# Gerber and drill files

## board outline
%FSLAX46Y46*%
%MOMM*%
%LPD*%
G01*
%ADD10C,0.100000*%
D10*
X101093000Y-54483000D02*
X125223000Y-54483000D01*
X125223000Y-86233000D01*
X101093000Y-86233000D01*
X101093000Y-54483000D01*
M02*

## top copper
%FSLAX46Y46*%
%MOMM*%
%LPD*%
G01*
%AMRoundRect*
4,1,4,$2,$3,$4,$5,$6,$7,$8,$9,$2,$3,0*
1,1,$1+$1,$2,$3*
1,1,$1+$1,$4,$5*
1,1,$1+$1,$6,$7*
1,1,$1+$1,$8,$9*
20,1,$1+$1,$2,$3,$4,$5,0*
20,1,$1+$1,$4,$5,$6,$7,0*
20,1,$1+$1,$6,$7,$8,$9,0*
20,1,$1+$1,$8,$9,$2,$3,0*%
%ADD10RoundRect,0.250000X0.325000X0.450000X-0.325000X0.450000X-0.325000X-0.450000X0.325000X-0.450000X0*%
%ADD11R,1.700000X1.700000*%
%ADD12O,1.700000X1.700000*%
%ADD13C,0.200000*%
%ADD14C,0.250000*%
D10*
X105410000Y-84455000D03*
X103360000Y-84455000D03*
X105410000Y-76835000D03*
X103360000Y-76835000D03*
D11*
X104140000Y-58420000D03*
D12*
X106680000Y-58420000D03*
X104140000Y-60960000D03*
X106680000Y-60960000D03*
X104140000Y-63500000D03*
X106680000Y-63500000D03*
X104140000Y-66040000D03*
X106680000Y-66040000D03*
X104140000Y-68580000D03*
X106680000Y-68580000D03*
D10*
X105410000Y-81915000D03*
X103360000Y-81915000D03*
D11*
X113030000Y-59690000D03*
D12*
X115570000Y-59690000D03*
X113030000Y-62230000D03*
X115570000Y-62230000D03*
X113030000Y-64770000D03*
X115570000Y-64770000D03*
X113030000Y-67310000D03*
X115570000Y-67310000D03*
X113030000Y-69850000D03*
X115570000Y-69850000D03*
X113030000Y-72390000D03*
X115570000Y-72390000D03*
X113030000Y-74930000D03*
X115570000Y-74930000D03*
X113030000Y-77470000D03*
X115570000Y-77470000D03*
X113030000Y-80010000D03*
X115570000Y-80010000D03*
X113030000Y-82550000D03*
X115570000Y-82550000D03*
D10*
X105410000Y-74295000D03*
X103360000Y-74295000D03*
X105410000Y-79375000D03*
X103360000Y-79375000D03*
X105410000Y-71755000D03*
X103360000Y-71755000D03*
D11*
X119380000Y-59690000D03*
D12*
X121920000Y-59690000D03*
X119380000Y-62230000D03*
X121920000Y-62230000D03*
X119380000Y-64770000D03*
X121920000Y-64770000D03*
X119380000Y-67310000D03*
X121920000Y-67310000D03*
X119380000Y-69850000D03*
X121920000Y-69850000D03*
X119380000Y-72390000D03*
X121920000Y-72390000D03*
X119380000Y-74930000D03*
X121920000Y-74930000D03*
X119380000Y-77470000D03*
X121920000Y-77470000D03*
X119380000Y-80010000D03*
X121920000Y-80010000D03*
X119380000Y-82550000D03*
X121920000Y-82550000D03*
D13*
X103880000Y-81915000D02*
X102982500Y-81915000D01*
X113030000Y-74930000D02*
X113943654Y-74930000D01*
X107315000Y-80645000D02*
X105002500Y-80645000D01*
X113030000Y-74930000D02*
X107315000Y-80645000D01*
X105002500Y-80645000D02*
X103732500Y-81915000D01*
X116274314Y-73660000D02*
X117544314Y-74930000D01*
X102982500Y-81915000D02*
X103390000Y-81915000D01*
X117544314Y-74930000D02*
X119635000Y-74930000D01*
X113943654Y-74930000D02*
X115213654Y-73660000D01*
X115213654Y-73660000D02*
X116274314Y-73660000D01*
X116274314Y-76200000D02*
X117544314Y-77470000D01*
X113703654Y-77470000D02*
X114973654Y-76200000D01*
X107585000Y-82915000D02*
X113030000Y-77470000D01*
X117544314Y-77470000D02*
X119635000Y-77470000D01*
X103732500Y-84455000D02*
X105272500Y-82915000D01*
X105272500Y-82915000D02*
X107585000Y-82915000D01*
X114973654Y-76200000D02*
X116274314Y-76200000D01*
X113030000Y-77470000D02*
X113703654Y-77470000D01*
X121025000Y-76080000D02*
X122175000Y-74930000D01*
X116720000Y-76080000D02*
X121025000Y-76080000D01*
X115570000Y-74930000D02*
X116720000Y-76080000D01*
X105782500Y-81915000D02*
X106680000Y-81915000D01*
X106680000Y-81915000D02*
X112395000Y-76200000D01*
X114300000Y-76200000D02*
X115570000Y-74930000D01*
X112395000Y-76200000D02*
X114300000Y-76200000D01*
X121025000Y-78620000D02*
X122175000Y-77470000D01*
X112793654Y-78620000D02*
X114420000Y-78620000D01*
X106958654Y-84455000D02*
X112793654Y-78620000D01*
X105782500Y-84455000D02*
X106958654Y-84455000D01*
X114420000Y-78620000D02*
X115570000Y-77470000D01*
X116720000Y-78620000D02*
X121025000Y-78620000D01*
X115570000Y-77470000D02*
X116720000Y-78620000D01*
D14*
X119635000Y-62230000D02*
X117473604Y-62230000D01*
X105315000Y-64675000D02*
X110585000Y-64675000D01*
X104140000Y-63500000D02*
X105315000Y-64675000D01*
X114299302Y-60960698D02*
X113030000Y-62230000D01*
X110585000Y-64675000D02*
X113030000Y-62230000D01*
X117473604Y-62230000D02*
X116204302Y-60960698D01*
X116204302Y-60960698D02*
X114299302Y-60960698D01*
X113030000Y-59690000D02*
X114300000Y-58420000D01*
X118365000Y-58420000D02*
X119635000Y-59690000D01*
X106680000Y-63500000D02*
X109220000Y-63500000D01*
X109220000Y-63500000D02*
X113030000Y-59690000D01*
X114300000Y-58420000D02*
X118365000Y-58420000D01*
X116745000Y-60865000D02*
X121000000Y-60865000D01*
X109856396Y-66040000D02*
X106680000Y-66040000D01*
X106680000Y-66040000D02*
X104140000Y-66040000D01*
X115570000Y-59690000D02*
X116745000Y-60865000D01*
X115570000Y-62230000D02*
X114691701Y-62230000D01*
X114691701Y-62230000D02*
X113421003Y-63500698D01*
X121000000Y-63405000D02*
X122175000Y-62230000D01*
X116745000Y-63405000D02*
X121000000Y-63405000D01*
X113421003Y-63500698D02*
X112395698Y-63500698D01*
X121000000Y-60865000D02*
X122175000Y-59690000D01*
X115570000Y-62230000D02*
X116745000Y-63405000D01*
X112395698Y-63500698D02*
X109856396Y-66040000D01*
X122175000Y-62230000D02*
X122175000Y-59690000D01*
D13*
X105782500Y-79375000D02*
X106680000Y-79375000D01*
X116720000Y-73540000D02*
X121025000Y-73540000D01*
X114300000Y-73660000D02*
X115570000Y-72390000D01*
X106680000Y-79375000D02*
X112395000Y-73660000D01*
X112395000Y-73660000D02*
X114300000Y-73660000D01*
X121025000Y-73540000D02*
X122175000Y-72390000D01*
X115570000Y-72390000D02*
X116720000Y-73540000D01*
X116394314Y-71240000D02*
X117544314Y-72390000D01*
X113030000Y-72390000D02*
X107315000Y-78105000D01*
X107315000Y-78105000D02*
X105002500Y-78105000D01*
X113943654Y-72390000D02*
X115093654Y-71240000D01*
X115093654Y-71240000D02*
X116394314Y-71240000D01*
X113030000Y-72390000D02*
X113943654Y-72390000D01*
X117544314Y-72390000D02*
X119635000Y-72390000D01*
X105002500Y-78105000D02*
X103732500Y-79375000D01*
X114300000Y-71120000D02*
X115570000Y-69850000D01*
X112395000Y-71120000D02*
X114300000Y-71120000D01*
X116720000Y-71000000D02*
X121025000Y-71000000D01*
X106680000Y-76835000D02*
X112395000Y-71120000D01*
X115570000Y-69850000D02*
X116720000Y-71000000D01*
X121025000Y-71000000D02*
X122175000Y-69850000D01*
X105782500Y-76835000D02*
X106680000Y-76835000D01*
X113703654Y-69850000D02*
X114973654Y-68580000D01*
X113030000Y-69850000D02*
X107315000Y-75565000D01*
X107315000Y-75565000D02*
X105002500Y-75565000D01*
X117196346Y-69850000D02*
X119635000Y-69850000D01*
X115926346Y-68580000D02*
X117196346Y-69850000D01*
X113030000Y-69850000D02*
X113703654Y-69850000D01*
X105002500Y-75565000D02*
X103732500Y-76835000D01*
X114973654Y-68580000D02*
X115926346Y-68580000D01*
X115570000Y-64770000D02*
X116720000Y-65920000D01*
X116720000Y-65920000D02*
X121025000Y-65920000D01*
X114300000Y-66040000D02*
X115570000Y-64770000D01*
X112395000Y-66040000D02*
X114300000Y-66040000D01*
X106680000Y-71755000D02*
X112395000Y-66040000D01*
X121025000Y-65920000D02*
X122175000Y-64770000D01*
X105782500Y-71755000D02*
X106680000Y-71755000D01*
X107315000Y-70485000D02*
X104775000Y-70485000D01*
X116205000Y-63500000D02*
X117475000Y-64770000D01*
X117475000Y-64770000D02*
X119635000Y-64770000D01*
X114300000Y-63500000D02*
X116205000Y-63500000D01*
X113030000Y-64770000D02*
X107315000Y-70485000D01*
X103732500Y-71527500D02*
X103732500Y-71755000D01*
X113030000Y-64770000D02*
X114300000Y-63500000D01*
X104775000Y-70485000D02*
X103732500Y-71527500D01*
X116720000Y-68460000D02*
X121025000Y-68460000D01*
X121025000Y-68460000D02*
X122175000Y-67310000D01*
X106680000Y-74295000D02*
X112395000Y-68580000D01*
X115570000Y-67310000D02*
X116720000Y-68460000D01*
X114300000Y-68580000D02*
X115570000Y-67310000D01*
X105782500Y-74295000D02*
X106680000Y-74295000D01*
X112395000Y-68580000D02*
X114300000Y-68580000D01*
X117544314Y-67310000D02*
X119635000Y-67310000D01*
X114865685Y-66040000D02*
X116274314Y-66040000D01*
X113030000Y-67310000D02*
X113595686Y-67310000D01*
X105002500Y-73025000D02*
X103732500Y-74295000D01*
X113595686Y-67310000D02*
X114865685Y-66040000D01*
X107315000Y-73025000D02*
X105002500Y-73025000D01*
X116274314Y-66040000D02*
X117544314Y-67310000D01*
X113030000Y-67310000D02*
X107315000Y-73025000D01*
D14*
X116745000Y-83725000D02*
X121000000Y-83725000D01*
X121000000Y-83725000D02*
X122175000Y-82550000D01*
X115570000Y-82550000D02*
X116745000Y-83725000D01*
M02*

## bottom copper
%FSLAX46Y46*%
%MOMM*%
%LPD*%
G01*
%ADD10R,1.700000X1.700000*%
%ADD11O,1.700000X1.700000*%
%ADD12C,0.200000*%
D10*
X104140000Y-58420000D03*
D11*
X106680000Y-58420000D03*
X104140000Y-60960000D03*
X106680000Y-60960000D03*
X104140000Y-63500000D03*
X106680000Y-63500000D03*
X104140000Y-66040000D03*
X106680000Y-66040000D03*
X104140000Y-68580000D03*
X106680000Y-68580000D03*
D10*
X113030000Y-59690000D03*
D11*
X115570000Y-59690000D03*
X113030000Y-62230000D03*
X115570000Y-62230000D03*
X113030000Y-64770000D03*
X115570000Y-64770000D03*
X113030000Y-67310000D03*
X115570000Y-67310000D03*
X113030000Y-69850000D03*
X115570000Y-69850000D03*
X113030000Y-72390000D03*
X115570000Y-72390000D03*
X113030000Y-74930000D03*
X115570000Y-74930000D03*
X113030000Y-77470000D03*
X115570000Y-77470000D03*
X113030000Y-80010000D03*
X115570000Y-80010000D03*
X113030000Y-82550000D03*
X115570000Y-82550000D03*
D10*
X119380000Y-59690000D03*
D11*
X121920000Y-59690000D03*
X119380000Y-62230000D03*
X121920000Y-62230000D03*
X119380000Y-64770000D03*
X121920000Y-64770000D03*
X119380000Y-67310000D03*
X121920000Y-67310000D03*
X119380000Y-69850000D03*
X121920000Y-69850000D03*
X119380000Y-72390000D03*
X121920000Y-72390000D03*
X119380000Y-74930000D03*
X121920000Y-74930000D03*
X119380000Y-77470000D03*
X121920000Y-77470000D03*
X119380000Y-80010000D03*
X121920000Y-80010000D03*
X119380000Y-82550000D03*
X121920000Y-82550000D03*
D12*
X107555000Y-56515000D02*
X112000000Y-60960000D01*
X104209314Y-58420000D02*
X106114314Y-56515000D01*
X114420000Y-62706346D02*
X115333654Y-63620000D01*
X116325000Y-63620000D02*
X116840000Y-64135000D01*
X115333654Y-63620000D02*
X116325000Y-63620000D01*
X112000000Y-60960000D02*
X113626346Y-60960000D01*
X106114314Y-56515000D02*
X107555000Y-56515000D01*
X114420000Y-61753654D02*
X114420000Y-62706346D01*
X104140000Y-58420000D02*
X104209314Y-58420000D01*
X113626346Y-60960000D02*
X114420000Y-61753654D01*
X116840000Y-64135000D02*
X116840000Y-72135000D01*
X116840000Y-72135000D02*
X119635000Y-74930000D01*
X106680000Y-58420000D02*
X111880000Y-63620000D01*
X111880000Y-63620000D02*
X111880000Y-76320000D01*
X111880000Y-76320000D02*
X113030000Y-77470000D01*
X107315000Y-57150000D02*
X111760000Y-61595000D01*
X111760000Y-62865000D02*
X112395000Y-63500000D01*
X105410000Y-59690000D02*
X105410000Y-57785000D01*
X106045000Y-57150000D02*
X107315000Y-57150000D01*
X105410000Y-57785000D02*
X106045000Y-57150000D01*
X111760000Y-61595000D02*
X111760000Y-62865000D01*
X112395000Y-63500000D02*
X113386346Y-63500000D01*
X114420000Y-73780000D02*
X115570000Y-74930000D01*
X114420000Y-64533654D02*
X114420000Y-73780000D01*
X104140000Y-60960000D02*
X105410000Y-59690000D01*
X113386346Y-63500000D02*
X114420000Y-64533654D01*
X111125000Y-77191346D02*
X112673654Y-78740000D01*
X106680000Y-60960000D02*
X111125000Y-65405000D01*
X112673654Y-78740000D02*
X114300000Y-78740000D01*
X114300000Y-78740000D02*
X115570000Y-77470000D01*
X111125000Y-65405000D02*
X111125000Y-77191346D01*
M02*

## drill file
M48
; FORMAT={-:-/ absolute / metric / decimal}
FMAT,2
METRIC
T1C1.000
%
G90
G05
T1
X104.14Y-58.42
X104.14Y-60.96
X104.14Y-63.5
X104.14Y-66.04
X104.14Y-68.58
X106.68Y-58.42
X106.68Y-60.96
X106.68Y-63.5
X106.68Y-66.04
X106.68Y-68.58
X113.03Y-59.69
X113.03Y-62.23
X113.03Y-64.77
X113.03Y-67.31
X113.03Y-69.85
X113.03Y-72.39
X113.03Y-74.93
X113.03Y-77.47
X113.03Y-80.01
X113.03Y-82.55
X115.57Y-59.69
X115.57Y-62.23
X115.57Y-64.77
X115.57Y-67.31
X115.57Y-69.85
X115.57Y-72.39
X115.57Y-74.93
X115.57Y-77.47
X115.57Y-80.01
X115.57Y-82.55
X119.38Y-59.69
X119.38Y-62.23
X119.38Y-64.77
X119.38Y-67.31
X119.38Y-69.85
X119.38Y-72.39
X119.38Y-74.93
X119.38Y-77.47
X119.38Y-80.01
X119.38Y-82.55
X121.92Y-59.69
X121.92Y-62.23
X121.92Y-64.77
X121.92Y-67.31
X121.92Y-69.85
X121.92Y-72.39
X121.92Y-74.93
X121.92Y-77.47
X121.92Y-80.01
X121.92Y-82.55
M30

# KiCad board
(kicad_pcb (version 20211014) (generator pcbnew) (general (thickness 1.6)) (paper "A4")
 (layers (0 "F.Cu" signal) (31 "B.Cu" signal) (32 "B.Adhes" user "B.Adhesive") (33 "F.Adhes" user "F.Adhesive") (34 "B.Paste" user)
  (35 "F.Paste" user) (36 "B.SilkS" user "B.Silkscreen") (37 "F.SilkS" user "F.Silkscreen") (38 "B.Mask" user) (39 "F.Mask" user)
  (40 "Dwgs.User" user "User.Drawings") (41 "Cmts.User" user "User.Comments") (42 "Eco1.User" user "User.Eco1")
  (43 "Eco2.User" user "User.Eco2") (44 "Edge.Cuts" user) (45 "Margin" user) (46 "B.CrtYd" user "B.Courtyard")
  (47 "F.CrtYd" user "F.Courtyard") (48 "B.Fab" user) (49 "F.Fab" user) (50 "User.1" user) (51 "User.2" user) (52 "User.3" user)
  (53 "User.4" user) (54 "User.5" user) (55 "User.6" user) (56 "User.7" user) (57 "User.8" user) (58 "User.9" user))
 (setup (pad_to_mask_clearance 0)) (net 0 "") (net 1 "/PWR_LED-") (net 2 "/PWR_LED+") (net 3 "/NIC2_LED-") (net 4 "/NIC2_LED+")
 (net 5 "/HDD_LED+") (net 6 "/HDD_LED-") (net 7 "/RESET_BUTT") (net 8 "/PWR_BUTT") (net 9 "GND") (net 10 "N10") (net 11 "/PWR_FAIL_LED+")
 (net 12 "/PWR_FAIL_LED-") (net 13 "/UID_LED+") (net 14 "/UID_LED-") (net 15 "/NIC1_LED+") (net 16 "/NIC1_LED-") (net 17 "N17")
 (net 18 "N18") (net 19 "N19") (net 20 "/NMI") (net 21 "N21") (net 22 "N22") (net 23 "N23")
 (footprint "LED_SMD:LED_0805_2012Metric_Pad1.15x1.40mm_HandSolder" (layer "F.Cu") (at 104.385 84.455 180)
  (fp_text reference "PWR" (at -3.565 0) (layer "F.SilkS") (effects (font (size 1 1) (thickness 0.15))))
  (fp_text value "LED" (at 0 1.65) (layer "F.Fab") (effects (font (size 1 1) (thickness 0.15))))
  (pad "1" smd roundrect (at -1.025 0 180) (size 1.15 1.4) (layers "F.Cu" "F.Paste" "F.Mask") (roundrect_rratio 0.217391)
   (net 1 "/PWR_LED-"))
  (pad "2" smd roundrect (at 1.025 0 180) (size 1.15 1.4) (layers "F.Cu" "F.Paste" "F.Mask") (roundrect_rratio 0.217391) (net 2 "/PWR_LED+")))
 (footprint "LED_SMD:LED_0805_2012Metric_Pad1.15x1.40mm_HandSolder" (layer "F.Cu") (at 104.385 76.835 180)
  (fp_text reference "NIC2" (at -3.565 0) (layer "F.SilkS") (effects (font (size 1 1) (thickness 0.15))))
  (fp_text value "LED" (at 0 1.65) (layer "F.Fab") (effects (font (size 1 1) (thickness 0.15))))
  (pad "1" smd roundrect (at -1.025 0 180) (size 1.15 1.4) (layers "F.Cu" "F.Paste" "F.Mask") (roundrect_rratio 0.217391)
   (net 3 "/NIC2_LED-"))
  (pad "2" smd roundrect (at 1.025 0 180) (size 1.15 1.4) (layers "F.Cu" "F.Paste" "F.Mask") (roundrect_rratio 0.217391)
   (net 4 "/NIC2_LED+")))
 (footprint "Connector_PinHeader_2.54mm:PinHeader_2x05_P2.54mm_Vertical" (layer "F.Cu") (at 104.14 58.42)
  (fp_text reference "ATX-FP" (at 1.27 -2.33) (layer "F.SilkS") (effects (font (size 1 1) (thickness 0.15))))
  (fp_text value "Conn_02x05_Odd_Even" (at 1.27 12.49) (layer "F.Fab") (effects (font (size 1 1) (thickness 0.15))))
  (pad "1" thru_hole rect (at 0 0) (size 1.7 1.7) (drill 1) (layers *.Cu *.Mask) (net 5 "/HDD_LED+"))
  (pad "2" thru_hole oval (at 2.54 0) (size 1.7 1.7) (drill 1) (layers *.Cu *.Mask) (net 2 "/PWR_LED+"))
  (pad "3" thru_hole oval (at 0 2.54) (size 1.7 1.7) (drill 1) (layers *.Cu *.Mask) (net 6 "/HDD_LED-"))
  (pad "4" thru_hole oval (at 2.54 2.54) (size 1.7 1.7) (drill 1) (layers *.Cu *.Mask) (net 1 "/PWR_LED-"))
  (pad "5" thru_hole oval (at 0 5.08) (size 1.7 1.7) (drill 1) (layers *.Cu *.Mask) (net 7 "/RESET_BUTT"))
  (pad "6" thru_hole oval (at 2.54 5.08) (size 1.7 1.7) (drill 1) (layers *.Cu *.Mask) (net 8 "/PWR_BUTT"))
  (pad "7" thru_hole oval (at 0 7.62) (size 1.7 1.7) (drill 1) (layers *.Cu *.Mask) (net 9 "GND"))
  (pad "8" thru_hole oval (at 2.54 7.62) (size 1.7 1.7) (drill 1) (layers *.Cu *.Mask) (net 9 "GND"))
  (pad "9" thru_hole oval (at 0 10.16) (size 1.7 1.7) (drill 1) (layers *.Cu *.Mask) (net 9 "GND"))
  (pad "10" thru_hole oval (at 2.54 10.16) (size 1.7 1.7) (drill 1) (layers *.Cu *.Mask) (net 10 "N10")))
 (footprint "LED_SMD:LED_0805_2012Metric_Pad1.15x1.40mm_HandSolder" (layer "F.Cu") (at 104.385 81.915 180)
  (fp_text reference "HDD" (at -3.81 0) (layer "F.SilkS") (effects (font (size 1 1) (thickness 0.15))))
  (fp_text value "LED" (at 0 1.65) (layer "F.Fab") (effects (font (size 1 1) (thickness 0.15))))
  (pad "1" smd roundrect (at -1.025 0 180) (size 1.15 1.4) (layers "F.Cu" "F.Paste" "F.Mask") (roundrect_rratio 0.217391)
   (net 6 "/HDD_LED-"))
  (pad "2" smd roundrect (at 1.025 0 180) (size 1.15 1.4) (layers "F.Cu" "F.Paste" "F.Mask") (roundrect_rratio 0.217391) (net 5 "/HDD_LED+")))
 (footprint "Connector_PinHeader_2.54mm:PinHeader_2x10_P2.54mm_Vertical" (layer "F.Cu") (at 113.03 59.69)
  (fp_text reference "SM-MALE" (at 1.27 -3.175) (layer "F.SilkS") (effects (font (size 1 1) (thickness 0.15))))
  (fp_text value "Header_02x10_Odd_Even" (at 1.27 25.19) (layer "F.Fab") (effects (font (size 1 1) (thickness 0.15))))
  (pad "1" thru_hole rect (at 0 0) (size 1.7 1.7) (drill 1) (layers *.Cu *.Mask) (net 8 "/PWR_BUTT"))
  (pad "2" thru_hole oval (at 2.54 0) (size 1.7 1.7) (drill 1) (layers *.Cu *.Mask) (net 9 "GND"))
  (pad "3" thru_hole oval (at 0 2.54) (size 1.7 1.7) (drill 1) (layers *.Cu *.Mask) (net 7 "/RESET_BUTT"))
  (pad "4" thru_hole oval (at 2.54 2.54) (size 1.7 1.7) (drill 1) (layers *.Cu *.Mask) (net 9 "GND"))
  (pad "5" thru_hole oval (at 0 5.08) (size 1.7 1.7) (drill 1) (layers *.Cu *.Mask) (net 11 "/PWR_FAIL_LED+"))
  (pad "6" thru_hole oval (at 2.54 5.08) (size 1.7 1.7) (drill 1) (layers *.Cu *.Mask) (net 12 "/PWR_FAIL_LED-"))
  (pad "7" thru_hole oval (at 0 7.62) (size 1.7 1.7) (drill 1) (layers *.Cu *.Mask) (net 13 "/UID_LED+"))
  (pad "8" thru_hole oval (at 2.54 7.62) (size 1.7 1.7) (drill 1) (layers *.Cu *.Mask) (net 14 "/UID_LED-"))
  (pad "9" thru_hole oval (at 0 10.16) (size 1.7 1.7) (drill 1) (layers *.Cu *.Mask) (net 4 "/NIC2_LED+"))
  (pad "10" thru_hole oval (at 2.54 10.16) (size 1.7 1.7) (drill 1) (layers *.Cu *.Mask) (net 3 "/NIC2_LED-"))
  (pad "11" thru_hole oval (at 0 12.7) (size 1.7 1.7) (drill 1) (layers *.Cu *.Mask) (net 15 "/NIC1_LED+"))
  (pad "12" thru_hole oval (at 2.54 12.7) (size 1.7 1.7) (drill 1) (layers *.Cu *.Mask) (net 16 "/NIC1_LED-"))
  (pad "13" thru_hole oval (at 0 15.24) (size 1.7 1.7) (drill 1) (layers *.Cu *.Mask) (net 5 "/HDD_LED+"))
  (pad "14" thru_hole oval (at 2.54 15.24) (size 1.7 1.7) (drill 1) (layers *.Cu *.Mask) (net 6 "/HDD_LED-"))
  (pad "15" thru_hole oval (at 0 17.78) (size 1.7 1.7) (drill 1) (layers *.Cu *.Mask) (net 2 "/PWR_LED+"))
  (pad "16" thru_hole oval (at 2.54 17.78) (size 1.7 1.7) (drill 1) (layers *.Cu *.Mask) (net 1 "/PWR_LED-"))
  (pad "17" thru_hole oval (at 0 20.32) (size 1.7 1.7) (drill 1) (layers *.Cu *.Mask) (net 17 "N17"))
  (pad "18" thru_hole oval (at 2.54 20.32) (size 1.7 1.7) (drill 1) (layers *.Cu *.Mask) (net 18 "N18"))
  (pad "19" thru_hole oval (at 0 22.86) (size 1.7 1.7) (drill 1) (layers *.Cu *.Mask) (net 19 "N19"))
  (pad "20" thru_hole oval (at 2.54 22.86) (size 1.7 1.7) (drill 1) (layers *.Cu *.Mask) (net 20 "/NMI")))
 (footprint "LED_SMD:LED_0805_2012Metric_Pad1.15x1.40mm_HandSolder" (layer "F.Cu") (at 104.385 74.295 180)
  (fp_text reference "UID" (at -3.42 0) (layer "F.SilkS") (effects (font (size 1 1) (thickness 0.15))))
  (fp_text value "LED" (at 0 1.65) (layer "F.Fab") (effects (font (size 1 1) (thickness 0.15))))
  (pad "1" smd roundrect (at -1.025 0 180) (size 1.15 1.4) (layers "F.Cu" "F.Paste" "F.Mask") (roundrect_rratio 0.217391)
   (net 14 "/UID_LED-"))
  (pad "2" smd roundrect (at 1.025 0 180) (size 1.15 1.4) (layers "F.Cu" "F.Paste" "F.Mask") (roundrect_rratio 0.217391)
   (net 13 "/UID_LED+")))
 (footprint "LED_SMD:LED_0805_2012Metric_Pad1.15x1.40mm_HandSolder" (layer "F.Cu") (at 104.385 79.375 180)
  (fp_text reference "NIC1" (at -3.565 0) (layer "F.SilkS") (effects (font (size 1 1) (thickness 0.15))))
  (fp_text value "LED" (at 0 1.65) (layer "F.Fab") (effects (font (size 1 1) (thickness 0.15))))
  (pad "1" smd roundrect (at -1.025 0 180) (size 1.15 1.4) (layers "F.Cu" "F.Paste" "F.Mask") (roundrect_rratio 0.217391)
   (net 16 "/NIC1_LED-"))
  (pad "2" smd roundrect (at 1.025 0 180) (size 1.15 1.4) (layers "F.Cu" "F.Paste" "F.Mask") (roundrect_rratio 0.217391)
   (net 15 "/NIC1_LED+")))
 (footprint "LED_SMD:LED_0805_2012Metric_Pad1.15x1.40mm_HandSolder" (layer "F.Cu") (at 104.385 71.755 180)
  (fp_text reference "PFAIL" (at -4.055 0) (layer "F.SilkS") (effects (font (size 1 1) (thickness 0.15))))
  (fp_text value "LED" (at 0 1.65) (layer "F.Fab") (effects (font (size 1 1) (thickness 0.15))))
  (pad "1" smd roundrect (at -1.025 0 180) (size 1.15 1.4) (layers "F.Cu" "F.Paste" "F.Mask") (roundrect_rratio 0.217391)
   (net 12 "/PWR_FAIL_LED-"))
  (pad "2" smd roundrect (at 1.025 0 180) (size 1.15 1.4) (layers "F.Cu" "F.Paste" "F.Mask") (roundrect_rratio 0.217391)
   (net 11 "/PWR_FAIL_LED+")))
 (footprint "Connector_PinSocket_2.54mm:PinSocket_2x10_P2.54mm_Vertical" (layer "B.Cu") (at 119.38 59.69 180)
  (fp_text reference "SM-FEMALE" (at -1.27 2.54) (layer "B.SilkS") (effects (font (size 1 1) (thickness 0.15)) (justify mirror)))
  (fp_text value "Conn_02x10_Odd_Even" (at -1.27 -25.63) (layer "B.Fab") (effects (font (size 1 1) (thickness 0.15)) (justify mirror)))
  (pad "1" thru_hole rect (at 0 0 180) (size 1.7 1.7) (drill 1) (layers *.Cu *.Mask) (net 8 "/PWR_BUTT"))
  (pad "2" thru_hole oval (at -2.54 0 180) (size 1.7 1.7) (drill 1) (layers *.Cu *.Mask) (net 9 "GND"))
  (pad "3" thru_hole oval (at 0 -2.54 180) (size 1.7 1.7) (drill 1) (layers *.Cu *.Mask) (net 7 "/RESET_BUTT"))
  (pad "4" thru_hole oval (at -2.54 -2.54 180) (size 1.7 1.7) (drill 1) (layers *.Cu *.Mask) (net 9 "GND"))
  (pad "5" thru_hole oval (at 0 -5.08 180) (size 1.7 1.7) (drill 1) (layers *.Cu *.Mask) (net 11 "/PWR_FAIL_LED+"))
  (pad "6" thru_hole oval (at -2.54 -5.08 180) (size 1.7 1.7) (drill 1) (layers *.Cu *.Mask) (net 12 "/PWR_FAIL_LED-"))
  (pad "7" thru_hole oval (at 0 -7.62 180) (size 1.7 1.7) (drill 1) (layers *.Cu *.Mask) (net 13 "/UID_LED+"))
  (pad "8" thru_hole oval (at -2.54 -7.62 180) (size 1.7 1.7) (drill 1) (layers *.Cu *.Mask) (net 14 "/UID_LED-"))
  (pad "9" thru_hole oval (at 0 -10.16 180) (size 1.7 1.7) (drill 1) (layers *.Cu *.Mask) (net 4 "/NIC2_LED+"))
  (pad "10" thru_hole oval (at -2.54 -10.16 180) (size 1.7 1.7) (drill 1) (layers *.Cu *.Mask) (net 3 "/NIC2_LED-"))
  (pad "11" thru_hole oval (at 0 -12.7 180) (size 1.7 1.7) (drill 1) (layers *.Cu *.Mask) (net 15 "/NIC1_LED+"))
  (pad "12" thru_hole oval (at -2.54 -12.7 180) (size 1.7 1.7) (drill 1) (layers *.Cu *.Mask) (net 16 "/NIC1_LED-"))
  (pad "13" thru_hole oval (at 0 -15.24 180) (size 1.7 1.7) (drill 1) (layers *.Cu *.Mask) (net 5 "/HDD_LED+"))
  (pad "14" thru_hole oval (at -2.54 -15.24 180) (size 1.7 1.7) (drill 1) (layers *.Cu *.Mask) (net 6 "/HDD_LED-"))
  (pad "15" thru_hole oval (at 0 -17.78 180) (size 1.7 1.7) (drill 1) (layers *.Cu *.Mask) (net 2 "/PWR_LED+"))
  (pad "16" thru_hole oval (at -2.54 -17.78 180) (size 1.7 1.7) (drill 1) (layers *.Cu *.Mask) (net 1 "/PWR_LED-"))
  (pad "17" thru_hole oval (at 0 -20.32 180) (size 1.7 1.7) (drill 1) (layers *.Cu *.Mask) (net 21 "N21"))
  (pad "18" thru_hole oval (at -2.54 -20.32 180) (size 1.7 1.7) (drill 1) (layers *.Cu *.Mask) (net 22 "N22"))
  (pad "19" thru_hole oval (at 0 -22.86 180) (size 1.7 1.7) (drill 1) (layers *.Cu *.Mask) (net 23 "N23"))
  (pad "20" thru_hole oval (at -2.54 -22.86 180) (size 1.7 1.7) (drill 1) (layers *.Cu *.Mask) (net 20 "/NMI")))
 (gr_rect (start 125.223 54.483) (end 101.093 86.233) (layer "Edge.Cuts") (width 0.1) (fill none))
 (segment (start 103.88 81.915) (end 102.9825 81.915) (width 0.2) (layer "F.Cu") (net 5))
 (segment (start 113.03 74.93) (end 113.943654 74.93) (width 0.2) (layer "F.Cu") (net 5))
 (segment (start 107.315 80.645) (end 105.0025 80.645) (width 0.2) (layer "F.Cu") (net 5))
 (segment (start 113.03 74.93) (end 107.315 80.645) (width 0.2) (layer "F.Cu") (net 5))
 (segment (start 105.0025 80.645) (end 103.7325 81.915) (width 0.2) (layer "F.Cu") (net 5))
 (segment (start 116.274314 73.66) (end 117.544314 74.93) (width 0.2) (layer "F.Cu") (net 5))
 (segment (start 102.9825 81.915) (end 103.39 81.915) (width 0.2) (layer "F.Cu") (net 5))
 (segment (start 117.544314 74.93) (end 119.635 74.93) (width 0.2) (layer "F.Cu") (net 5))
 (segment (start 113.943654 74.93) (end 115.213654 73.66) (width 0.2) (layer "F.Cu") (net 5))
 (segment (start 115.213654 73.66) (end 116.274314 73.66) (width 0.2) (layer "F.Cu") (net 5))
 (segment (start 107.555 56.515) (end 112 60.96) (width 0.2) (layer "B.Cu") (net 5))
 (segment (start 104.209314 58.42) (end 106.114314 56.515) (width 0.2) (layer "B.Cu") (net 5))
 (segment (start 114.42 62.706346) (end 115.333654 63.62) (width 0.2) (layer "B.Cu") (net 5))
 (segment (start 116.325 63.62) (end 116.84 64.135) (width 0.2) (layer "B.Cu") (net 5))
 (segment (start 115.333654 63.62) (end 116.325 63.62) (width 0.2) (layer "B.Cu") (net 5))
 (segment (start 112 60.96) (end 113.626346 60.96) (width 0.2) (layer "B.Cu") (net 5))
 (segment (start 106.114314 56.515) (end 107.555 56.515) (width 0.2) (layer "B.Cu") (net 5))
 (segment (start 114.42 61.753654) (end 114.42 62.706346) (width 0.2) (layer "B.Cu") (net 5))
 (segment (start 104.14 58.42) (end 104.209314 58.42) (width 0.2) (layer "B.Cu") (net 5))
 (segment (start 113.626346 60.96) (end 114.42 61.753654) (width 0.2) (layer "B.Cu") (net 5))
 (segment (start 116.84 64.135) (end 116.84 72.135) (width 0.2) (layer "B.Cu") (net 5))
 (segment (start 116.84 72.135) (end 119.635 74.93) (width 0.2) (layer "B.Cu") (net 5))
 (segment (start 116.274314 76.2) (end 117.544314 77.47) (width 0.2) (layer "F.Cu") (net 2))
 (segment (start 113.703654 77.47) (end 114.973654 76.2) (width 0.2) (layer "F.Cu") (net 2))
 (segment (start 107.585 82.915) (end 113.03 77.47) (width 0.2) (layer "F.Cu") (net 2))
 (segment (start 117.544314 77.47) (end 119.635 77.47) (width 0.2) (layer "F.Cu") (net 2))
 (segment (start 103.7325 84.455) (end 105.2725 82.915) (width 0.2) (layer "F.Cu") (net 2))
 (segment (start 105.2725 82.915) (end 107.585 82.915) (width 0.2) (layer "F.Cu") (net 2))
 (segment (start 114.973654 76.2) (end 116.274314 76.2) (width 0.2) (layer "F.Cu") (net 2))
 (segment (start 113.03 77.47) (end 113.703654 77.47) (width 0.2) (layer "F.Cu") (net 2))
 (segment (start 106.68 58.42) (end 111.88 63.62) (width 0.2) (layer "B.Cu") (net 2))
 (segment (start 111.88 63.62) (end 111.88 76.32) (width 0.2) (layer "B.Cu") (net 2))
 (segment (start 111.88 76.32) (end 113.03 77.47) (width 0.2) (layer "B.Cu") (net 2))
 (segment (start 121.025 76.08) (end 122.175 74.93) (width 0.2) (layer "F.Cu") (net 6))
 (segment (start 116.72 76.08) (end 121.025 76.08) (width 0.2) (layer "F.Cu") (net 6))
 (segment (start 115.57 74.93) (end 116.72 76.08) (width 0.2) (layer "F.Cu") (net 6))
 (segment (start 105.7825 81.915) (end 106.68 81.915) (width 0.2) (layer "F.Cu") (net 6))
 (segment (start 106.68 81.915) (end 112.395 76.2) (width 0.2) (layer "F.Cu") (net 6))
 (segment (start 114.3 76.2) (end 115.57 74.93) (width 0.2) (layer "F.Cu") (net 6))
 (segment (start 112.395 76.2) (end 114.3 76.2) (width 0.2) (layer "F.Cu") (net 6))
 (segment (start 107.315 57.15) (end 111.76 61.595) (width 0.2) (layer "B.Cu") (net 6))
 (segment (start 111.76 62.865) (end 112.395 63.5) (width 0.2) (layer "B.Cu") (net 6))
 (segment (start 105.41 59.69) (end 105.41 57.785) (width 0.2) (layer "B.Cu") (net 6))
 (segment (start 106.045 57.15) (end 107.315 57.15) (width 0.2) (layer "B.Cu") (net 6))
 (segment (start 105.41 57.785) (end 106.045 57.15) (width 0.2) (layer "B.Cu") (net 6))
 (segment (start 111.76 61.595) (end 111.76 62.865) (width 0.2) (layer "B.Cu") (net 6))
 (segment (start 112.395 63.5) (end 113.386346 63.5) (width 0.2) (layer "B.Cu") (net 6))
 (segment (start 114.42 73.78) (end 115.57 74.93) (width 0.2) (layer "B.Cu") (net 6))
 (segment (start 114.42 64.533654) (end 114.42 73.78) (width 0.2) (layer "B.Cu") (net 6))
 (segment (start 104.14 60.96) (end 105.41 59.69) (width 0.2) (layer "B.Cu") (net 6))
 (segment (start 113.386346 63.5) (end 114.42 64.533654) (width 0.2) (layer "B.Cu") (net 6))
 (segment (start 121.025 78.62) (end 122.175 77.47) (width 0.2) (layer "F.Cu") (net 1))
 (segment (start 112.793654 78.62) (end 114.42 78.62) (width 0.2) (layer "F.Cu") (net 1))
 (segment (start 106.958654 84.455) (end 112.793654 78.62) (width 0.2) (layer "F.Cu") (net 1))
 (segment (start 105.7825 84.455) (end 106.958654 84.455) (width 0.2) (layer "F.Cu") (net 1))
 (segment (start 114.42 78.62) (end 115.57 77.47) (width 0.2) (layer "F.Cu") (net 1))
 (segment (start 116.72 78.62) (end 121.025 78.62) (width 0.2) (layer "F.Cu") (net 1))
 (segment (start 115.57 77.47) (end 116.72 78.62) (width 0.2) (layer "F.Cu") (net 1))
 (segment (start 111.125 77.191346) (end 112.673654 78.74) (width 0.2) (layer "B.Cu") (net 1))
 (segment (start 106.68 60.96) (end 111.125 65.405) (width 0.2) (layer "B.Cu") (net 1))
 (segment (start 112.673654 78.74) (end 114.3 78.74) (width 0.2) (layer "B.Cu") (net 1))
 (segment (start 114.3 78.74) (end 115.57 77.47) (width 0.2) (layer "B.Cu") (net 1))
 (segment (start 111.125 65.405) (end 111.125 77.191346) (width 0.2) (layer "B.Cu") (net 1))
 (segment (start 119.635 62.23) (end 117.473604 62.23) (width 0.25) (layer "F.Cu") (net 7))
 (segment (start 105.315 64.675) (end 110.585 64.675) (width 0.25) (layer "F.Cu") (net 7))
 (segment (start 104.14 63.5) (end 105.315 64.675) (width 0.25) (layer "F.Cu") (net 7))
 (segment (start 114.299302 60.960698) (end 113.03 62.23) (width 0.25) (layer "F.Cu") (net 7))
 (segment (start 110.585 64.675) (end 113.03 62.23) (width 0.25) (layer "F.Cu") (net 7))
 (segment (start 117.473604 62.23) (end 116.204302 60.960698) (width 0.25) (layer "F.Cu") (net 7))
 (segment (start 116.204302 60.960698) (end 114.299302 60.960698) (width 0.25) (layer "F.Cu") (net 7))
 (segment (start 113.03 59.69) (end 114.3 58.42) (width 0.25) (layer "F.Cu") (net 8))
 (segment (start 118.365 58.42) (end 119.635 59.69) (width 0.25) (layer "F.Cu") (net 8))
 (segment (start 106.68 63.5) (end 109.22 63.5) (width 0.25) (layer "F.Cu") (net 8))
 (segment (start 109.22 63.5) (end 113.03 59.69) (width 0.25) (layer "F.Cu") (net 8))
 (segment (start 114.3 58.42) (end 118.365 58.42) (width 0.25) (layer "F.Cu") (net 8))
 (segment (start 116.745 60.865) (end 121 60.865) (width 0.25) (layer "F.Cu") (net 9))
 (segment (start 109.856396 66.04) (end 106.68 66.04) (width 0.25) (layer "F.Cu") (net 9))
 (segment (start 106.68 66.04) (end 104.14 66.04) (width 0.25) (layer "F.Cu") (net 9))
 (segment (start 115.57 59.69) (end 116.745 60.865) (width 0.25) (layer "F.Cu") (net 9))
 (segment (start 115.57 62.23) (end 114.691701 62.23) (width 0.25) (layer "F.Cu") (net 9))
 (segment (start 114.691701 62.23) (end 113.421003 63.500698) (width 0.25) (layer "F.Cu") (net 9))
 (segment (start 121 63.405) (end 122.175 62.23) (width 0.25) (layer "F.Cu") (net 9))
 (segment (start 116.745 63.405) (end 121 63.405) (width 0.25) (layer "F.Cu") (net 9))
 (segment (start 113.421003 63.500698) (end 112.395698 63.500698) (width 0.25) (layer "F.Cu") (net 9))
 (segment (start 121 60.865) (end 122.175 59.69) (width 0.25) (layer "F.Cu") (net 9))
 (segment (start 115.57 62.23) (end 116.745 63.405) (width 0.25) (layer "F.Cu") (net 9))
 (segment (start 112.395698 63.500698) (end 109.856396 66.04) (width 0.25) (layer "F.Cu") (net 9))
 (segment (start 122.175 62.23) (end 122.175 59.69) (width 0.25) (layer "F.Cu") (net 9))
 (segment (start 105.7825 79.375) (end 106.68 79.375) (width 0.2) (layer "F.Cu") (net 16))
 (segment (start 116.72 73.54) (end 121.025 73.54) (width 0.2) (layer "F.Cu") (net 16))
 (segment (start 114.3 73.66) (end 115.57 72.39) (width 0.2) (layer "F.Cu") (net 16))
 (segment (start 106.68 79.375) (end 112.395 73.66) (width 0.2) (layer "F.Cu") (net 16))
 (segment (start 112.395 73.66) (end 114.3 73.66) (width 0.2) (layer "F.Cu") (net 16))
 (segment (start 121.025 73.54) (end 122.175 72.39) (width 0.2) (layer "F.Cu") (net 16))
 (segment (start 115.57 72.39) (end 116.72 73.54) (width 0.2) (layer "F.Cu") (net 16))
 (segment (start 116.394314 71.24) (end 117.544314 72.39) (width 0.2) (layer "F.Cu") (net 15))
 (segment (start 113.03 72.39) (end 107.315 78.105) (width 0.2) (layer "F.Cu") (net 15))
 (segment (start 107.315 78.105) (end 105.0025 78.105) (width 0.2) (layer "F.Cu") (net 15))
 (segment (start 113.943654 72.39) (end 115.093654 71.24) (width 0.2) (layer "F.Cu") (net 15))
 (segment (start 115.093654 71.24) (end 116.394314 71.24) (width 0.2) (layer "F.Cu") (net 15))
 (segment (start 113.03 72.39) (end 113.943654 72.39) (width 0.2) (layer "F.Cu") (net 15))
 (segment (start 117.544314 72.39) (end 119.635 72.39) (width 0.2) (layer "F.Cu") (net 15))
 (segment (start 105.0025 78.105) (end 103.7325 79.375) (width 0.2) (layer "F.Cu") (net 15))
 (segment (start 114.3 71.12) (end 115.57 69.85) (width 0.2) (layer "F.Cu") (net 3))
 (segment (start 112.395 71.12) (end 114.3 71.12) (width 0.2) (layer "F.Cu") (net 3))
 (segment (start 116.72 71) (end 121.025 71) (width 0.2) (layer "F.Cu") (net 3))
 (segment (start 106.68 76.835) (end 112.395 71.12) (width 0.2) (layer "F.Cu") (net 3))
 (segment (start 115.57 69.85) (end 116.72 71) (width 0.2) (layer "F.Cu") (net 3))
 (segment (start 121.025 71) (end 122.175 69.85) (width 0.2) (layer "F.Cu") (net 3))
 (segment (start 105.7825 76.835) (end 106.68 76.835) (width 0.2) (layer "F.Cu") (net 3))
 (segment (start 113.703654 69.85) (end 114.973654 68.58) (width 0.2) (layer "F.Cu") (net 4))
 (segment (start 113.03 69.85) (end 107.315 75.565) (width 0.2) (layer "F.Cu") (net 4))
 (segment (start 107.315 75.565) (end 105.0025 75.565) (width 0.2) (layer "F.Cu") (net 4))
 (segment (start 117.196346 69.85) (end 119.635 69.85) (width 0.2) (layer "F.Cu") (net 4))
 (segment (start 115.926346 68.58) (end 117.196346 69.85) (width 0.2) (layer "F.Cu") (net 4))
 (segment (start 113.03 69.85) (end 113.703654 69.85) (width 0.2) (layer "F.Cu") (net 4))
 (segment (start 105.0025 75.565) (end 103.7325 76.835) (width 0.2) (layer "F.Cu") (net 4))
 (segment (start 114.973654 68.58) (end 115.926346 68.58) (width 0.2) (layer "F.Cu") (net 4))
 (segment (start 115.57 64.77) (end 116.72 65.92) (width 0.2) (layer "F.Cu") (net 12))
 (segment (start 116.72 65.92) (end 121.025 65.92) (width 0.2) (layer "F.Cu") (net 12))
 (segment (start 114.3 66.04) (end 115.57 64.77) (width 0.2) (layer "F.Cu") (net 12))
 (segment (start 112.395 66.04) (end 114.3 66.04) (width 0.2) (layer "F.Cu") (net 12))
 (segment (start 106.68 71.755) (end 112.395 66.04) (width 0.2) (layer "F.Cu") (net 12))
 (segment (start 121.025 65.92) (end 122.175 64.77) (width 0.2) (layer "F.Cu") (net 12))
 (segment (start 105.7825 71.755) (end 106.68 71.755) (width 0.2) (layer "F.Cu") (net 12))
 (segment (start 107.315 70.485) (end 104.775 70.485) (width 0.2) (layer "F.Cu") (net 11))
 (segment (start 116.205 63.5) (end 117.475 64.77) (width 0.2) (layer "F.Cu") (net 11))
 (segment (start 117.475 64.77) (end 119.635 64.77) (width 0.2) (layer "F.Cu") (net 11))
 (segment (start 114.3 63.5) (end 116.205 63.5) (width 0.2) (layer "F.Cu") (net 11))
 (segment (start 113.03 64.77) (end 107.315 70.485) (width 0.2) (layer "F.Cu") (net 11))
 (segment (start 103.7325 71.5275) (end 103.7325 71.755) (width 0.2) (layer "F.Cu") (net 11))
 (segment (start 113.03 64.77) (end 114.3 63.5) (width 0.2) (layer "F.Cu") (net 11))
 (segment (start 104.775 70.485) (end 103.7325 71.5275) (width 0.2) (layer "F.Cu") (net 11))
 (segment (start 116.72 68.46) (end 121.025 68.46) (width 0.2) (layer "F.Cu") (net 14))
 (segment (start 121.025 68.46) (end 122.175 67.31) (width 0.2) (layer "F.Cu") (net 14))
 (segment (start 106.68 74.295) (end 112.395 68.58) (width 0.2) (layer "F.Cu") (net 14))
 (segment (start 115.57 67.31) (end 116.72 68.46) (width 0.2) (layer "F.Cu") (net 14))
 (segment (start 114.3 68.58) (end 115.57 67.31) (width 0.2) (layer "F.Cu") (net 14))
 (segment (start 105.7825 74.295) (end 106.68 74.295) (width 0.2) (layer "F.Cu") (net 14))
 (segment (start 112.395 68.58) (end 114.3 68.58) (width 0.2) (layer "F.Cu") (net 14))
 (segment (start 117.544314 67.31) (end 119.635 67.31) (width 0.2) (layer "F.Cu") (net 13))
 (segment (start 114.865685 66.04) (end 116.274314 66.04) (width 0.2) (layer "F.Cu") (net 13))
 (segment (start 113.03 67.31) (end 113.595686 67.31) (width 0.2) (layer "F.Cu") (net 13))
 (segment (start 105.0025 73.025) (end 103.7325 74.295) (width 0.2) (layer "F.Cu") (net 13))
 (segment (start 113.595686 67.31) (end 114.865685 66.04) (width 0.2) (layer "F.Cu") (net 13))
 (segment (start 107.315 73.025) (end 105.0025 73.025) (width 0.2) (layer "F.Cu") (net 13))
 (segment (start 116.274314 66.04) (end 117.544314 67.31) (width 0.2) (layer "F.Cu") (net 13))
 (segment (start 113.03 67.31) (end 107.315 73.025) (width 0.2) (layer "F.Cu") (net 13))
 (segment (start 116.745 83.725) (end 121 83.725) (width 0.25) (layer "F.Cu") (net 20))
 (segment (start 121 83.725) (end 122.175 82.55) (width 0.25) (layer "F.Cu") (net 20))
 (segment (start 115.57 82.55) (end 116.745 83.725) (width 0.25) (layer "F.Cu") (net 20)))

